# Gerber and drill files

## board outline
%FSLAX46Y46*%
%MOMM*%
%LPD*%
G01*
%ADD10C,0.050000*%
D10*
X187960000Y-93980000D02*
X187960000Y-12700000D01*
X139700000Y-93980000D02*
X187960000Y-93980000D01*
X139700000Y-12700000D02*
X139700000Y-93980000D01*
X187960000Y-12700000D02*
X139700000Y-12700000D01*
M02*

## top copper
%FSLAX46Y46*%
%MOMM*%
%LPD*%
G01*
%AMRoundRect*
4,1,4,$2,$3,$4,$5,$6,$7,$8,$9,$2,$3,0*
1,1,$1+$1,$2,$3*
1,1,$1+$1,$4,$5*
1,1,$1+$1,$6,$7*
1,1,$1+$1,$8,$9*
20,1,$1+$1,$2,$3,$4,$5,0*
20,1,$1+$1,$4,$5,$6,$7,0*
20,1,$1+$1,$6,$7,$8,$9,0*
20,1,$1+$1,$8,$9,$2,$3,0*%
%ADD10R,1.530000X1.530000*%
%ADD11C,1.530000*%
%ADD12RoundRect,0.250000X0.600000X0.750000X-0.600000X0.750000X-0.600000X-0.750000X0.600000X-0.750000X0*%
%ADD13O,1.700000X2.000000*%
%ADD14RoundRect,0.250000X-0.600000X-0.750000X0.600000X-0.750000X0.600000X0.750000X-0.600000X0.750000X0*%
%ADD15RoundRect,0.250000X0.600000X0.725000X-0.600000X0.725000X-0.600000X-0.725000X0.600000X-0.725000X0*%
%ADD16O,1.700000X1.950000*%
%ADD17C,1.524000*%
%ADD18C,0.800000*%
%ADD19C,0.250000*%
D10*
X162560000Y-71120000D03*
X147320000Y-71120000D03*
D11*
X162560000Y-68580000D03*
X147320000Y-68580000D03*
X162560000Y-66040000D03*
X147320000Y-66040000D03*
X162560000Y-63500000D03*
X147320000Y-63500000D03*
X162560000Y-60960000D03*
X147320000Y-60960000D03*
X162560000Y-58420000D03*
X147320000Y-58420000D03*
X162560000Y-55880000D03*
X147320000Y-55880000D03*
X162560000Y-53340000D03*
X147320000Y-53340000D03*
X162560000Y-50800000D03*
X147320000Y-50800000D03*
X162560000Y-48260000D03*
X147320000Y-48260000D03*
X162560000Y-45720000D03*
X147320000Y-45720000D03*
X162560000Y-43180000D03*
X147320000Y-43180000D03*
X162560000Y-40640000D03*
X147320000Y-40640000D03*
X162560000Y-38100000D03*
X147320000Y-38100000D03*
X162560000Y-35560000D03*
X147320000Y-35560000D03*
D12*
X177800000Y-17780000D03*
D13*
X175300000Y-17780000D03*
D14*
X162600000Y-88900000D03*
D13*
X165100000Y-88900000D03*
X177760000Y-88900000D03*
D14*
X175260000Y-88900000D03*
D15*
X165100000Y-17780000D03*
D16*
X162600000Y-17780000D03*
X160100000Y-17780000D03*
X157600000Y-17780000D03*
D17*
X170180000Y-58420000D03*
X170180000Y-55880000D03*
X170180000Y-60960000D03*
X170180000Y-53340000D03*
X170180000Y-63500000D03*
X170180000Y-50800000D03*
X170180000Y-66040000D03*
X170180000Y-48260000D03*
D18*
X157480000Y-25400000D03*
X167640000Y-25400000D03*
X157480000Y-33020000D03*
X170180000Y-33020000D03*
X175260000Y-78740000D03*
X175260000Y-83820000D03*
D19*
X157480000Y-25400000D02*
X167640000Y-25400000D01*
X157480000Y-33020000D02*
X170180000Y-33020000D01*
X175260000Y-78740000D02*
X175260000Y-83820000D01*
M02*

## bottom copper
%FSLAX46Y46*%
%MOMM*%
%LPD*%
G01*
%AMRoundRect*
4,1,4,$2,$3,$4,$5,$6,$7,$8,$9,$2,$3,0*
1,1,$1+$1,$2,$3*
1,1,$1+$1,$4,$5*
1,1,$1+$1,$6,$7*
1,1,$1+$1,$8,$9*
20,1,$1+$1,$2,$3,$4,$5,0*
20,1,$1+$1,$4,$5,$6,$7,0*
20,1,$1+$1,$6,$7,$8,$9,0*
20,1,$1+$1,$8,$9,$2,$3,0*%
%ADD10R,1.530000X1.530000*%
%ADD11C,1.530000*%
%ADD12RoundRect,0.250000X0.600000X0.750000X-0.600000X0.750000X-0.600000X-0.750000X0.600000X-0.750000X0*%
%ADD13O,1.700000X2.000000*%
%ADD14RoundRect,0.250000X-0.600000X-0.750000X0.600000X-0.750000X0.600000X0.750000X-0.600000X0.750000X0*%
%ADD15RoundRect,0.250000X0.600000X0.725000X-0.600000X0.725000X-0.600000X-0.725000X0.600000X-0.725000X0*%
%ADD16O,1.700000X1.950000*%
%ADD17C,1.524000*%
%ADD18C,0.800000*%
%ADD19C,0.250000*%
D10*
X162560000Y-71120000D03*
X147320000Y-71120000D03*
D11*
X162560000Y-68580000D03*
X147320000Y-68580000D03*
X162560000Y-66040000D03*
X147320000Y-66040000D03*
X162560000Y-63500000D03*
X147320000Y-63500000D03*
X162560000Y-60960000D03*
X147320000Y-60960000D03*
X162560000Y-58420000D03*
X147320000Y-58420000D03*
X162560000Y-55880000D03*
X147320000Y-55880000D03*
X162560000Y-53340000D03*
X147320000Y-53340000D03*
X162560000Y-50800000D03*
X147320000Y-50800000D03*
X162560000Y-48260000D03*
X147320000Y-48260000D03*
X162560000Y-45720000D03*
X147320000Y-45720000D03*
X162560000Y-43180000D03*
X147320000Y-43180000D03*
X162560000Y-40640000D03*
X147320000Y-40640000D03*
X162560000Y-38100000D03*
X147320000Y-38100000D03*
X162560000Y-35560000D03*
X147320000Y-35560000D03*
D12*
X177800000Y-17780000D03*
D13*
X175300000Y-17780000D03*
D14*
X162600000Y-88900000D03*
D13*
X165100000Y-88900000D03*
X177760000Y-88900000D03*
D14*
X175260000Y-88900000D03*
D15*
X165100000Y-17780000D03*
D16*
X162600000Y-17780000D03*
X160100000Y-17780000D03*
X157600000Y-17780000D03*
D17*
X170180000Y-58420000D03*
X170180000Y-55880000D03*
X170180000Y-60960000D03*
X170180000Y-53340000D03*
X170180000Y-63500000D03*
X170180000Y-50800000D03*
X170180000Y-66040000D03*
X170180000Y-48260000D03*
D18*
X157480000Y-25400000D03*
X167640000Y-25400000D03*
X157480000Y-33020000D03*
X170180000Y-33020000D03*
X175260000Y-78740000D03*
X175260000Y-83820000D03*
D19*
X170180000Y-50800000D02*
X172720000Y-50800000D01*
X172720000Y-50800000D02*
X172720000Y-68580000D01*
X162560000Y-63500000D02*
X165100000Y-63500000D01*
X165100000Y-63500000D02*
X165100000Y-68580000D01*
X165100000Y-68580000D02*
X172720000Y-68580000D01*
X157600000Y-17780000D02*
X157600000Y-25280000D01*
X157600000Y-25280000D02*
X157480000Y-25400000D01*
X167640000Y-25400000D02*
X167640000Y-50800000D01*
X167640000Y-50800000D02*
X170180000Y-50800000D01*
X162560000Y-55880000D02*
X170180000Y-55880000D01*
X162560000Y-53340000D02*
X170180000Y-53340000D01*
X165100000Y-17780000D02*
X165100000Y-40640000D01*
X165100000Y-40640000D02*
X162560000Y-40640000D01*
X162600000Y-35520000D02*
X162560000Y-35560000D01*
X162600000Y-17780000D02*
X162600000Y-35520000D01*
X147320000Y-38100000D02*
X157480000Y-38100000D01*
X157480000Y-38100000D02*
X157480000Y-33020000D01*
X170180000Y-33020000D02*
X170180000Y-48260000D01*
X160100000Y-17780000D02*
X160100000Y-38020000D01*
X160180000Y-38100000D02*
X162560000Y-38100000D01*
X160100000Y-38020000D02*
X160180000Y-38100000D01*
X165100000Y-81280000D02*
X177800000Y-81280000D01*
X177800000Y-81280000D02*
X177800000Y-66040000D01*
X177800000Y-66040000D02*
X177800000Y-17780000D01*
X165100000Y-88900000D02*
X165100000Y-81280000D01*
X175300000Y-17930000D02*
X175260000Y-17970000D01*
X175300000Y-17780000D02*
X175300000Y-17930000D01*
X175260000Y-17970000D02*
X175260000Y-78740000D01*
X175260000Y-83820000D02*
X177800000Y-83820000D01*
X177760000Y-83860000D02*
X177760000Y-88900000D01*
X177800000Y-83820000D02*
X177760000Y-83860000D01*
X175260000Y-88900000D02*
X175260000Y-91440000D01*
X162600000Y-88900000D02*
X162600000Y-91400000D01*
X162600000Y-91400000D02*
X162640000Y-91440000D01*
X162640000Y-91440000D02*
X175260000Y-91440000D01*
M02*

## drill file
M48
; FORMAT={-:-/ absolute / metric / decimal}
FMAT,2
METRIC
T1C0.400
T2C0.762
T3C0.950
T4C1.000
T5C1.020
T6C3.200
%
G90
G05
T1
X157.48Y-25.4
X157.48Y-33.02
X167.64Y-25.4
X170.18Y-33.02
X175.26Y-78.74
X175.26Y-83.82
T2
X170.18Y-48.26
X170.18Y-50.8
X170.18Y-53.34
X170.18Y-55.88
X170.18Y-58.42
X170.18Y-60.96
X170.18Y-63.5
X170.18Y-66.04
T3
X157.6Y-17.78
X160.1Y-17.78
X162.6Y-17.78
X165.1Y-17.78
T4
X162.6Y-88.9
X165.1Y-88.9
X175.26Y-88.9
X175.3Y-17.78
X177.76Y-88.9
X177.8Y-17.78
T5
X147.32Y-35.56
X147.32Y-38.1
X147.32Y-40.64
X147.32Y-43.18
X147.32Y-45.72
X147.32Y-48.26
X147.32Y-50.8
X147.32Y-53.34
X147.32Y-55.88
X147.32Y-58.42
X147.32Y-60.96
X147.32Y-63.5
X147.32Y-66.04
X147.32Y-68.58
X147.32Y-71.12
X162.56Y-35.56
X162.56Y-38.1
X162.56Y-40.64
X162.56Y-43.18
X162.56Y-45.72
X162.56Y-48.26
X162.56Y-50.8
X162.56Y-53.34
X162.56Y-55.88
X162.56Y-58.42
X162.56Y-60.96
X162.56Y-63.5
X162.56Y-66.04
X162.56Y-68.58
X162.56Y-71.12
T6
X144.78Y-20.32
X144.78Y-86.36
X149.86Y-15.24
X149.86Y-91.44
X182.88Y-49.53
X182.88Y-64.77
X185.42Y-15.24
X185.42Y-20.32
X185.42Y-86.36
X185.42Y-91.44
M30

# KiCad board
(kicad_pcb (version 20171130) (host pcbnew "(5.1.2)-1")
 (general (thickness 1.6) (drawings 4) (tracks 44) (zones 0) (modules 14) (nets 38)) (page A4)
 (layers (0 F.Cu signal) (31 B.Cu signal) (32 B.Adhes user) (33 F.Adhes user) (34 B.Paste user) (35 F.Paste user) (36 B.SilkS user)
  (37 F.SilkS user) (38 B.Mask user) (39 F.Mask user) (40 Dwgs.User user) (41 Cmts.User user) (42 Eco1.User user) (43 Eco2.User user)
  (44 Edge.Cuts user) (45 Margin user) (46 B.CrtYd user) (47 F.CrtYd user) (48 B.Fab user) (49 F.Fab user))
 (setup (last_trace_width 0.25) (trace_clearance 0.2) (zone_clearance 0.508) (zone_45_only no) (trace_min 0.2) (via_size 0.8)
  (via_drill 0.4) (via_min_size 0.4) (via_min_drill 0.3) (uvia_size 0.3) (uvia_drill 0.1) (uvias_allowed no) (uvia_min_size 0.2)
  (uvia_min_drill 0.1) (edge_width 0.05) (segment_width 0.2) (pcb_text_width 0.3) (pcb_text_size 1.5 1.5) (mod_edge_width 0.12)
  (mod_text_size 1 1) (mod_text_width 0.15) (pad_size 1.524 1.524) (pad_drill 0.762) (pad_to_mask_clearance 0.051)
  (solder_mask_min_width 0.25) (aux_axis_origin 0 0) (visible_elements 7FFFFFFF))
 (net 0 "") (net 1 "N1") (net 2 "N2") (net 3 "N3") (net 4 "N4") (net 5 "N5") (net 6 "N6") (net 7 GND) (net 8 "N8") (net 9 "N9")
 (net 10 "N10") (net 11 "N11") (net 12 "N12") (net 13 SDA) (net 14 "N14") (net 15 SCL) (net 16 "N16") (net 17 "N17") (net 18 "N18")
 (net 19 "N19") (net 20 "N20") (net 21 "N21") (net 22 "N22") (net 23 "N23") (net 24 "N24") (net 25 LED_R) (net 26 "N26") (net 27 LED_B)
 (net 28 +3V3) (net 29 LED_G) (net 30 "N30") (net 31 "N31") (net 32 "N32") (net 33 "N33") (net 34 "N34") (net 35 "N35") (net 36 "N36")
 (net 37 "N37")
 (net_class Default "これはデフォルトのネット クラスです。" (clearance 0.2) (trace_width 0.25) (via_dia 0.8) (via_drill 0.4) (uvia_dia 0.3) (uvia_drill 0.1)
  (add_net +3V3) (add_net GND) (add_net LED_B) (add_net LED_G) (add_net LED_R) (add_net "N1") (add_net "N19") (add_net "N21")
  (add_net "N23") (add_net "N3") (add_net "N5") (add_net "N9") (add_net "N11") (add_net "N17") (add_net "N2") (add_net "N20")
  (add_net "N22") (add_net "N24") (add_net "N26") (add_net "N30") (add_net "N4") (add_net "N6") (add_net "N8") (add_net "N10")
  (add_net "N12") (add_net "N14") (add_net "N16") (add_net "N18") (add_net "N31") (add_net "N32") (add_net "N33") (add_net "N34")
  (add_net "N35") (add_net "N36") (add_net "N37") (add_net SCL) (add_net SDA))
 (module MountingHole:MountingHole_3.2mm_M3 (layer F.Cu) (at 144.78 86.36)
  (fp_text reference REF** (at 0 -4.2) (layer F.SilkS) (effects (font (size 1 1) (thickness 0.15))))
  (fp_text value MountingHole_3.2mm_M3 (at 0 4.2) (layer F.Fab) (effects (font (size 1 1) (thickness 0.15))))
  (pad 1 np_thru_hole circle (at 0 0) (size 3.2 3.2) (drill 3.2) (layers *.Cu *.Mask)))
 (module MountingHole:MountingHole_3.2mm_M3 (layer F.Cu) (at 185.42 86.36)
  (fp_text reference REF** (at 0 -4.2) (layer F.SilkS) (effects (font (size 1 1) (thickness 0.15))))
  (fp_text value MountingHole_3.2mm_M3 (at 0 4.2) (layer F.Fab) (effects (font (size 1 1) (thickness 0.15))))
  (pad 1 np_thru_hole circle (at 0 0) (size 3.2 3.2) (drill 3.2) (layers *.Cu *.Mask)))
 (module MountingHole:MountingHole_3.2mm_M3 (layer F.Cu) (at 144.78 20.32)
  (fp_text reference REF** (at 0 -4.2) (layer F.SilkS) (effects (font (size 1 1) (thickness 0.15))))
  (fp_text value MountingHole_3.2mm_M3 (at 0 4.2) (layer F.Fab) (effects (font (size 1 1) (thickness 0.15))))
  (pad 1 np_thru_hole circle (at 0 0) (size 3.2 3.2) (drill 3.2) (layers *.Cu *.Mask)))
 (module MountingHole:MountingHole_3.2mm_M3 (layer F.Cu) (at 185.42 20.32)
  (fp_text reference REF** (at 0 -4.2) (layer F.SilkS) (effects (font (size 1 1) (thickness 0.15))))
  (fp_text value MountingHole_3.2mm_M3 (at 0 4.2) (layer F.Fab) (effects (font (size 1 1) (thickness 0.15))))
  (pad 1 np_thru_hole circle (at 0 0) (size 3.2 3.2) (drill 3.2) (layers *.Cu *.Mask)))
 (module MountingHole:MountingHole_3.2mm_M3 (layer F.Cu) (at 149.86 91.44)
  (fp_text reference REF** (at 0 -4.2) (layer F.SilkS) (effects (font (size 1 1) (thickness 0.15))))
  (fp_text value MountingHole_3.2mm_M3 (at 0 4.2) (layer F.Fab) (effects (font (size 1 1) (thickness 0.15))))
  (pad 1 np_thru_hole circle (at 0 0) (size 3.2 3.2) (drill 3.2) (layers *.Cu *.Mask)))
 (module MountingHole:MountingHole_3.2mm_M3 (layer F.Cu) (at 185.42 91.44)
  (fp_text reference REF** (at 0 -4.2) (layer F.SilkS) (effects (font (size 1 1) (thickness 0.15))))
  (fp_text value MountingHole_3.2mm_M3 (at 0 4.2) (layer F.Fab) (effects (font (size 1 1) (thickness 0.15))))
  (pad 1 np_thru_hole circle (at 0 0) (size 3.2 3.2) (drill 3.2) (layers *.Cu *.Mask)))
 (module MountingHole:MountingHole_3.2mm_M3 (layer F.Cu) (at 149.86 15.24)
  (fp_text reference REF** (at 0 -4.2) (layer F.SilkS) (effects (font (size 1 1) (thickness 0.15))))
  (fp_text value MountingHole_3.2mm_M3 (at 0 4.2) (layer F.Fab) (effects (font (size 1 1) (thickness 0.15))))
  (pad 1 np_thru_hole circle (at 0 0) (size 3.2 3.2) (drill 3.2) (layers *.Cu *.Mask)))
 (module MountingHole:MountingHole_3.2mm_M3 (layer F.Cu) (at 185.42 15.24)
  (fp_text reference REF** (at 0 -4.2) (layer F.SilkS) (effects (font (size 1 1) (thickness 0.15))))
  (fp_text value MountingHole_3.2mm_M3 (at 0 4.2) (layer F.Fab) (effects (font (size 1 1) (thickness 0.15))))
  (pad 1 np_thru_hole circle (at 0 0) (size 3.2 3.2) (drill 3.2) (layers *.Cu *.Mask)))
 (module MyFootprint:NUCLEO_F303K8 (layer F.Cu) (at 154.94 53.34 180)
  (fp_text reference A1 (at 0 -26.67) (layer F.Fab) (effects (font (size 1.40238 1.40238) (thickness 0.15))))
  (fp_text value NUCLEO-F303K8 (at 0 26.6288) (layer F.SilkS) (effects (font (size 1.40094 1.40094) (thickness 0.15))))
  (pad 3.1 thru_hole rect (at -7.62 -17.78 180) (size 1.53 1.53) (drill 1.02) (layers *.Cu *.Mask) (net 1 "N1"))
  (pad 4.1 thru_hole rect (at 7.62 -17.78 180) (size 1.53 1.53) (drill 1.02) (layers *.Cu *.Mask) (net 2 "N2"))
  (pad 3.2 thru_hole circle (at -7.62 -15.24 180) (size 1.53 1.53) (drill 1.02) (layers *.Cu *.Mask) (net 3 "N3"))
  (pad 4.2 thru_hole circle (at 7.62 -15.24 180) (size 1.53 1.53) (drill 1.02) (layers *.Cu *.Mask) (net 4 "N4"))
  (pad 3.3 thru_hole circle (at -7.62 -12.7 180) (size 1.53 1.53) (drill 1.02) (layers *.Cu *.Mask) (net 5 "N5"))
  (pad 4.3 thru_hole circle (at 7.62 -12.7 180) (size 1.53 1.53) (drill 1.02) (layers *.Cu *.Mask) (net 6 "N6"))
  (pad 3.4 thru_hole circle (at -7.62 -10.16 180) (size 1.53 1.53) (drill 1.02) (layers *.Cu *.Mask) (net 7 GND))
  (pad 4.4 thru_hole circle (at 7.62 -10.16 180) (size 1.53 1.53) (drill 1.02) (layers *.Cu *.Mask) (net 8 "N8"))
  (pad 3.5 thru_hole circle (at -7.62 -7.62 180) (size 1.53 1.53) (drill 1.02) (layers *.Cu *.Mask) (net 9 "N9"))
  (pad 4.5 thru_hole circle (at 7.62 -7.62 180) (size 1.53 1.53) (drill 1.02) (layers *.Cu *.Mask) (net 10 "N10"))
  (pad 3.6 thru_hole circle (at -7.62 -5.08 180) (size 1.53 1.53) (drill 1.02) (layers *.Cu *.Mask) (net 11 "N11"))
  (pad 4.6 thru_hole circle (at 7.62 -5.08 180) (size 1.53 1.53) (drill 1.02) (layers *.Cu *.Mask) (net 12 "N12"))
  (pad 3.7 thru_hole circle (at -7.62 -2.54 180) (size 1.53 1.53) (drill 1.02) (layers *.Cu *.Mask) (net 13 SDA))
  (pad 4.7 thru_hole circle (at 7.62 -2.54 180) (size 1.53 1.53) (drill 1.02) (layers *.Cu *.Mask) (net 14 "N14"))
  (pad 3.8 thru_hole circle (at -7.62 0 180) (size 1.53 1.53) (drill 1.02) (layers *.Cu *.Mask) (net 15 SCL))
  (pad 4.8 thru_hole circle (at 7.62 0 180) (size 1.53 1.53) (drill 1.02) (layers *.Cu *.Mask) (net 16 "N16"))
  (pad 3.9 thru_hole circle (at -7.62 2.54 180) (size 1.53 1.53) (drill 1.02) (layers *.Cu *.Mask) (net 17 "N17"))
  (pad 4.9 thru_hole circle (at 7.62 2.54 180) (size 1.53 1.53) (drill 1.02) (layers *.Cu *.Mask) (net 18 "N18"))
  (pad 3.10 thru_hole circle (at -7.62 5.08 180) (size 1.53 1.53) (drill 1.02) (layers *.Cu *.Mask) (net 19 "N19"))
  (pad 4.10 thru_hole circle (at 7.62 5.08 180) (size 1.53 1.53) (drill 1.02) (layers *.Cu *.Mask) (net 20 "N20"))
  (pad 3.11 thru_hole circle (at -7.62 7.62 180) (size 1.53 1.53) (drill 1.02) (layers *.Cu *.Mask) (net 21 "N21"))
  (pad 4.11 thru_hole circle (at 7.62 7.62 180) (size 1.53 1.53) (drill 1.02) (layers *.Cu *.Mask) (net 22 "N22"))
  (pad 3.12 thru_hole circle (at -7.62 10.16 180) (size 1.53 1.53) (drill 1.02) (layers *.Cu *.Mask) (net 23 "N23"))
  (pad 4.12 thru_hole circle (at 7.62 10.16 180) (size 1.53 1.53) (drill 1.02) (layers *.Cu *.Mask) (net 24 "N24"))
  (pad 3.13 thru_hole circle (at -7.62 12.7 180) (size 1.53 1.53) (drill 1.02) (layers *.Cu *.Mask) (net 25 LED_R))
  (pad 4.13 thru_hole circle (at 7.62 12.7 180) (size 1.53 1.53) (drill 1.02) (layers *.Cu *.Mask) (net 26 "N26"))
  (pad 3.14 thru_hole circle (at -7.62 15.24 180) (size 1.53 1.53) (drill 1.02) (layers *.Cu *.Mask) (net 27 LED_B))
  (pad 4.14 thru_hole circle (at 7.62 15.24 180) (size 1.53 1.53) (drill 1.02) (layers *.Cu *.Mask) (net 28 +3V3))
  (pad 3.15 thru_hole circle (at -7.62 17.78 180) (size 1.53 1.53) (drill 1.02) (layers *.Cu *.Mask) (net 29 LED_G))
  (pad 4.15 thru_hole circle (at 7.62 17.78 180) (size 1.53 1.53) (drill 1.02) (layers *.Cu *.Mask) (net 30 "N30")))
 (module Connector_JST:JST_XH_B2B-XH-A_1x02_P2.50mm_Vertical (layer F.Cu) (at 177.8 17.78 180)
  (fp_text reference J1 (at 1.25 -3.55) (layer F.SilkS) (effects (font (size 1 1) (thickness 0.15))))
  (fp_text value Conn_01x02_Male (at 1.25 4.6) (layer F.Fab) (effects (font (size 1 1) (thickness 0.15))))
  (pad 1 thru_hole roundrect (at 0 0 180) (size 1.7 2) (drill 1) (layers *.Cu *.Mask) (roundrect_rratio 0.147059) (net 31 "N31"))
  (pad 2 thru_hole oval (at 2.5 0 180) (size 1.7 2) (drill 1) (layers *.Cu *.Mask) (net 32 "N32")))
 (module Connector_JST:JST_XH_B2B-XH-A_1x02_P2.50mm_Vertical (layer F.Cu) (at 162.6 88.9)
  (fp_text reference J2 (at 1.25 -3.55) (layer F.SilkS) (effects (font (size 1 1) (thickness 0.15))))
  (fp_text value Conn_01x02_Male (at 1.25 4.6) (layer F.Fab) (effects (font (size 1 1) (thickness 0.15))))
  (pad 1 thru_hole roundrect (at 0 0) (size 1.7 2) (drill 1) (layers *.Cu *.Mask) (roundrect_rratio 0.147059) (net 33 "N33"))
  (pad 2 thru_hole oval (at 2.5 0) (size 1.7 2) (drill 1) (layers *.Cu *.Mask) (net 31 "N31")))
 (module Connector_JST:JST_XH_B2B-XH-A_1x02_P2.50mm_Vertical (layer F.Cu) (at 175.26 88.9)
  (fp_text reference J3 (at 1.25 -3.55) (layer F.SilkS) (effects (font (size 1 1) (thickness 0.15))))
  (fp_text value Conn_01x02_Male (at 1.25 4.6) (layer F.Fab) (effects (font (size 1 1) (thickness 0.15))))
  (pad 2 thru_hole oval (at 2.5 0) (size 1.7 2) (drill 1) (layers *.Cu *.Mask) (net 32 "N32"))
  (pad 1 thru_hole roundrect (at 0 0) (size 1.7 2) (drill 1) (layers *.Cu *.Mask) (roundrect_rratio 0.147059) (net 33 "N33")))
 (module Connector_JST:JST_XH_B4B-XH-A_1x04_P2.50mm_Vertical (layer F.Cu) (at 165.1 17.78 180)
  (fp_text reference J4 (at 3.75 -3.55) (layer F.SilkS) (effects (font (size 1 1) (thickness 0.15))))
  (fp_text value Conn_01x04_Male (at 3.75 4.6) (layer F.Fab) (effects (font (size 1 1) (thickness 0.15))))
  (pad 1 thru_hole roundrect (at 0 0 180) (size 1.7 1.95) (drill 0.95) (layers *.Cu *.Mask) (roundrect_rratio 0.147059) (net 25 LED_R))
  (pad 2 thru_hole oval (at 2.5 0 180) (size 1.7 1.95) (drill 0.95) (layers *.Cu *.Mask) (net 29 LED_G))
  (pad 3 thru_hole oval (at 5 0 180) (size 1.7 1.95) (drill 0.95) (layers *.Cu *.Mask) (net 27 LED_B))
  (pad 4 thru_hole oval (at 7.5 0 180) (size 1.7 1.95) (drill 0.95) (layers *.Cu *.Mask) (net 7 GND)))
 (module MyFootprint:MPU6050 (layer F.Cu) (at 175.26 58.42)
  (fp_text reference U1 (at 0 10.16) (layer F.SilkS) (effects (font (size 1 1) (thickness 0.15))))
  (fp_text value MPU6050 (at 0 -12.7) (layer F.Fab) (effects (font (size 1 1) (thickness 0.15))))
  (pad 5 thru_hole circle (at -5.08 0) (size 1.524 1.524) (drill 0.762) (layers *.Cu *.Mask) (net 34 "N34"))
  (pad 4 thru_hole circle (at -5.08 -2.54) (size 1.524 1.524) (drill 0.762) (layers *.Cu *.Mask) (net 13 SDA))
  (pad 6 thru_hole circle (at -5.08 2.54) (size 1.524 1.524) (drill 0.762) (layers *.Cu *.Mask) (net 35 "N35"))
  (pad 3 thru_hole circle (at -5.08 -5.08) (size 1.524 1.524) (drill 0.762) (layers *.Cu *.Mask) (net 15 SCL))
  (pad 7 thru_hole circle (at -5.08 5.08) (size 1.524 1.524) (drill 0.762) (layers *.Cu *.Mask) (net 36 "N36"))
  (pad 2 thru_hole circle (at -5.08 -7.62) (size 1.524 1.524) (drill 0.762) (layers *.Cu *.Mask) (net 7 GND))
  (pad 8 thru_hole circle (at -5.08 7.62) (size 1.524 1.524) (drill 0.762) (layers *.Cu *.Mask) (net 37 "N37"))
  (pad 1 thru_hole circle (at -5.08 -10.16) (size 1.524 1.524) (drill 0.762) (layers *.Cu *.Mask) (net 28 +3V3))
  (pad "" np_thru_hole circle (at 7.62 -8.89) (size 3.2 3.2) (drill 3.2) (layers *.Cu *.Mask))
  (pad "" np_thru_hole circle (at 7.62 6.35) (size 3.2 3.2) (drill 3.2) (layers *.Cu *.Mask)))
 (gr_line (start 187.96 93.98) (end 187.96 12.7) (layer Edge.Cuts) (width 0.05))
 (gr_line (start 139.7 93.98) (end 187.96 93.98) (layer Edge.Cuts) (width 0.05))
 (gr_line (start 139.7 12.7) (end 139.7 93.98) (layer Edge.Cuts) (width 0.05))
 (gr_line (start 187.96 12.7) (end 139.7 12.7) (layer Edge.Cuts) (width 0.05))
 (segment (start 170.18 50.8) (end 172.72 50.8) (width 0.25) (layer B.Cu) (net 7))
 (segment (start 172.72 50.8) (end 172.72 68.58) (width 0.25) (layer B.Cu) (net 7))
 (segment (start 162.56 63.5) (end 165.1 63.5) (width 0.25) (layer B.Cu) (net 7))
 (segment (start 165.1 63.5) (end 165.1 68.58) (width 0.25) (layer B.Cu) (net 7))
 (segment (start 165.1 68.58) (end 172.72 68.58) (width 0.25) (layer B.Cu) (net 7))
 (via (at 157.48 25.4) (size 0.8) (drill 0.4) (layers F.Cu B.Cu) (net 7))
 (segment (start 157.6 17.78) (end 157.6 25.28) (width 0.25) (layer B.Cu) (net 7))
 (segment (start 157.6 25.28) (end 157.48 25.4) (width 0.25) (layer B.Cu) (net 7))
 (via (at 167.64 25.4) (size 0.8) (drill 0.4) (layers F.Cu B.Cu) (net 7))
 (segment (start 157.48 25.4) (end 167.64 25.4) (width 0.25) (layer F.Cu) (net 7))
 (segment (start 167.64 25.4) (end 167.64 50.8) (width 0.25) (layer B.Cu) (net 7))
 (segment (start 167.64 50.8) (end 170.18 50.8) (width 0.25) (layer B.Cu) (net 7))
 (segment (start 162.56 55.88) (end 170.18 55.88) (width 0.25) (layer B.Cu) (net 13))
 (segment (start 162.56 53.34) (end 170.18 53.34) (width 0.25) (layer B.Cu) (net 15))
 (segment (start 165.1 17.78) (end 165.1 40.64) (width 0.25) (layer B.Cu) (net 25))
 (segment (start 165.1 40.64) (end 162.56 40.64) (width 0.25) (layer B.Cu) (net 25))
 (segment (start 162.6 35.52) (end 162.56 35.56) (width 0.25) (layer B.Cu) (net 29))
 (segment (start 162.6 17.78) (end 162.6 35.52) (width 0.25) (layer B.Cu) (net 29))
 (segment (start 147.32 38.1) (end 157.48 38.1) (width 0.25) (layer B.Cu) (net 28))
 (via (at 157.48 33.02) (size 0.8) (drill 0.4) (layers F.Cu B.Cu) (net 28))
 (segment (start 157.48 38.1) (end 157.48 33.02) (width 0.25) (layer B.Cu) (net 28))
 (via (at 170.18 33.02) (size 0.8) (drill 0.4) (layers F.Cu B.Cu) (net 28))
 (segment (start 157.48 33.02) (end 170.18 33.02) (width 0.25) (layer F.Cu) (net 28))
 (segment (start 170.18 33.02) (end 170.18 48.26) (width 0.25) (layer B.Cu) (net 28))
 (segment (start 160.1 17.78) (end 160.1 38.02) (width 0.25) (layer B.Cu) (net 27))
 (segment (start 160.18 38.1) (end 162.56 38.1) (width 0.25) (layer B.Cu) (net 27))
 (segment (start 160.1 38.02) (end 160.18 38.1) (width 0.25) (layer B.Cu) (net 27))
 (segment (start 165.1 81.28) (end 177.8 81.28) (width 0.25) (layer B.Cu) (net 31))
 (segment (start 177.8 81.28) (end 177.8 66.04) (width 0.25) (layer B.Cu) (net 31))
 (segment (start 177.8 66.04) (end 177.8 17.78) (width 0.25) (layer B.Cu) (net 31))
 (segment (start 165.1 88.9) (end 165.1 81.28) (width 0.25) (layer B.Cu) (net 31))
 (segment (start 175.3 17.93) (end 175.26 17.97) (width 0.25) (layer B.Cu) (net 32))
 (segment (start 175.3 17.78) (end 175.3 17.93) (width 0.25) (layer B.Cu) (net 32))
 (via (at 175.26 78.74) (size 0.8) (drill 0.4) (layers F.Cu B.Cu) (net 32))
 (segment (start 175.26 17.97) (end 175.26 78.74) (width 0.25) (layer B.Cu) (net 32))
 (via (at 175.26 83.82) (size 0.8) (drill 0.4) (layers F.Cu B.Cu) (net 32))
 (segment (start 175.26 78.74) (end 175.26 83.82) (width 0.25) (layer F.Cu) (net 32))
 (segment (start 175.26 83.82) (end 177.8 83.82) (width 0.25) (layer B.Cu) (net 32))
 (segment (start 177.76 83.86) (end 177.76 88.9) (width 0.25) (layer B.Cu) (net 32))
 (segment (start 177.8 83.82) (end 177.76 83.86) (width 0.25) (layer B.Cu) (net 32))
 (segment (start 175.26 88.9) (end 175.26 91.44) (width 0.25) (layer B.Cu) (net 33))
 (segment (start 162.6 88.9) (end 162.6 91.4) (width 0.25) (layer B.Cu) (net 33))
 (segment (start 162.6 91.4) (end 162.64 91.44) (width 0.25) (layer B.Cu) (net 33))
 (segment (start 162.64 91.44) (end 175.26 91.44) (width 0.25) (layer B.Cu) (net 33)))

